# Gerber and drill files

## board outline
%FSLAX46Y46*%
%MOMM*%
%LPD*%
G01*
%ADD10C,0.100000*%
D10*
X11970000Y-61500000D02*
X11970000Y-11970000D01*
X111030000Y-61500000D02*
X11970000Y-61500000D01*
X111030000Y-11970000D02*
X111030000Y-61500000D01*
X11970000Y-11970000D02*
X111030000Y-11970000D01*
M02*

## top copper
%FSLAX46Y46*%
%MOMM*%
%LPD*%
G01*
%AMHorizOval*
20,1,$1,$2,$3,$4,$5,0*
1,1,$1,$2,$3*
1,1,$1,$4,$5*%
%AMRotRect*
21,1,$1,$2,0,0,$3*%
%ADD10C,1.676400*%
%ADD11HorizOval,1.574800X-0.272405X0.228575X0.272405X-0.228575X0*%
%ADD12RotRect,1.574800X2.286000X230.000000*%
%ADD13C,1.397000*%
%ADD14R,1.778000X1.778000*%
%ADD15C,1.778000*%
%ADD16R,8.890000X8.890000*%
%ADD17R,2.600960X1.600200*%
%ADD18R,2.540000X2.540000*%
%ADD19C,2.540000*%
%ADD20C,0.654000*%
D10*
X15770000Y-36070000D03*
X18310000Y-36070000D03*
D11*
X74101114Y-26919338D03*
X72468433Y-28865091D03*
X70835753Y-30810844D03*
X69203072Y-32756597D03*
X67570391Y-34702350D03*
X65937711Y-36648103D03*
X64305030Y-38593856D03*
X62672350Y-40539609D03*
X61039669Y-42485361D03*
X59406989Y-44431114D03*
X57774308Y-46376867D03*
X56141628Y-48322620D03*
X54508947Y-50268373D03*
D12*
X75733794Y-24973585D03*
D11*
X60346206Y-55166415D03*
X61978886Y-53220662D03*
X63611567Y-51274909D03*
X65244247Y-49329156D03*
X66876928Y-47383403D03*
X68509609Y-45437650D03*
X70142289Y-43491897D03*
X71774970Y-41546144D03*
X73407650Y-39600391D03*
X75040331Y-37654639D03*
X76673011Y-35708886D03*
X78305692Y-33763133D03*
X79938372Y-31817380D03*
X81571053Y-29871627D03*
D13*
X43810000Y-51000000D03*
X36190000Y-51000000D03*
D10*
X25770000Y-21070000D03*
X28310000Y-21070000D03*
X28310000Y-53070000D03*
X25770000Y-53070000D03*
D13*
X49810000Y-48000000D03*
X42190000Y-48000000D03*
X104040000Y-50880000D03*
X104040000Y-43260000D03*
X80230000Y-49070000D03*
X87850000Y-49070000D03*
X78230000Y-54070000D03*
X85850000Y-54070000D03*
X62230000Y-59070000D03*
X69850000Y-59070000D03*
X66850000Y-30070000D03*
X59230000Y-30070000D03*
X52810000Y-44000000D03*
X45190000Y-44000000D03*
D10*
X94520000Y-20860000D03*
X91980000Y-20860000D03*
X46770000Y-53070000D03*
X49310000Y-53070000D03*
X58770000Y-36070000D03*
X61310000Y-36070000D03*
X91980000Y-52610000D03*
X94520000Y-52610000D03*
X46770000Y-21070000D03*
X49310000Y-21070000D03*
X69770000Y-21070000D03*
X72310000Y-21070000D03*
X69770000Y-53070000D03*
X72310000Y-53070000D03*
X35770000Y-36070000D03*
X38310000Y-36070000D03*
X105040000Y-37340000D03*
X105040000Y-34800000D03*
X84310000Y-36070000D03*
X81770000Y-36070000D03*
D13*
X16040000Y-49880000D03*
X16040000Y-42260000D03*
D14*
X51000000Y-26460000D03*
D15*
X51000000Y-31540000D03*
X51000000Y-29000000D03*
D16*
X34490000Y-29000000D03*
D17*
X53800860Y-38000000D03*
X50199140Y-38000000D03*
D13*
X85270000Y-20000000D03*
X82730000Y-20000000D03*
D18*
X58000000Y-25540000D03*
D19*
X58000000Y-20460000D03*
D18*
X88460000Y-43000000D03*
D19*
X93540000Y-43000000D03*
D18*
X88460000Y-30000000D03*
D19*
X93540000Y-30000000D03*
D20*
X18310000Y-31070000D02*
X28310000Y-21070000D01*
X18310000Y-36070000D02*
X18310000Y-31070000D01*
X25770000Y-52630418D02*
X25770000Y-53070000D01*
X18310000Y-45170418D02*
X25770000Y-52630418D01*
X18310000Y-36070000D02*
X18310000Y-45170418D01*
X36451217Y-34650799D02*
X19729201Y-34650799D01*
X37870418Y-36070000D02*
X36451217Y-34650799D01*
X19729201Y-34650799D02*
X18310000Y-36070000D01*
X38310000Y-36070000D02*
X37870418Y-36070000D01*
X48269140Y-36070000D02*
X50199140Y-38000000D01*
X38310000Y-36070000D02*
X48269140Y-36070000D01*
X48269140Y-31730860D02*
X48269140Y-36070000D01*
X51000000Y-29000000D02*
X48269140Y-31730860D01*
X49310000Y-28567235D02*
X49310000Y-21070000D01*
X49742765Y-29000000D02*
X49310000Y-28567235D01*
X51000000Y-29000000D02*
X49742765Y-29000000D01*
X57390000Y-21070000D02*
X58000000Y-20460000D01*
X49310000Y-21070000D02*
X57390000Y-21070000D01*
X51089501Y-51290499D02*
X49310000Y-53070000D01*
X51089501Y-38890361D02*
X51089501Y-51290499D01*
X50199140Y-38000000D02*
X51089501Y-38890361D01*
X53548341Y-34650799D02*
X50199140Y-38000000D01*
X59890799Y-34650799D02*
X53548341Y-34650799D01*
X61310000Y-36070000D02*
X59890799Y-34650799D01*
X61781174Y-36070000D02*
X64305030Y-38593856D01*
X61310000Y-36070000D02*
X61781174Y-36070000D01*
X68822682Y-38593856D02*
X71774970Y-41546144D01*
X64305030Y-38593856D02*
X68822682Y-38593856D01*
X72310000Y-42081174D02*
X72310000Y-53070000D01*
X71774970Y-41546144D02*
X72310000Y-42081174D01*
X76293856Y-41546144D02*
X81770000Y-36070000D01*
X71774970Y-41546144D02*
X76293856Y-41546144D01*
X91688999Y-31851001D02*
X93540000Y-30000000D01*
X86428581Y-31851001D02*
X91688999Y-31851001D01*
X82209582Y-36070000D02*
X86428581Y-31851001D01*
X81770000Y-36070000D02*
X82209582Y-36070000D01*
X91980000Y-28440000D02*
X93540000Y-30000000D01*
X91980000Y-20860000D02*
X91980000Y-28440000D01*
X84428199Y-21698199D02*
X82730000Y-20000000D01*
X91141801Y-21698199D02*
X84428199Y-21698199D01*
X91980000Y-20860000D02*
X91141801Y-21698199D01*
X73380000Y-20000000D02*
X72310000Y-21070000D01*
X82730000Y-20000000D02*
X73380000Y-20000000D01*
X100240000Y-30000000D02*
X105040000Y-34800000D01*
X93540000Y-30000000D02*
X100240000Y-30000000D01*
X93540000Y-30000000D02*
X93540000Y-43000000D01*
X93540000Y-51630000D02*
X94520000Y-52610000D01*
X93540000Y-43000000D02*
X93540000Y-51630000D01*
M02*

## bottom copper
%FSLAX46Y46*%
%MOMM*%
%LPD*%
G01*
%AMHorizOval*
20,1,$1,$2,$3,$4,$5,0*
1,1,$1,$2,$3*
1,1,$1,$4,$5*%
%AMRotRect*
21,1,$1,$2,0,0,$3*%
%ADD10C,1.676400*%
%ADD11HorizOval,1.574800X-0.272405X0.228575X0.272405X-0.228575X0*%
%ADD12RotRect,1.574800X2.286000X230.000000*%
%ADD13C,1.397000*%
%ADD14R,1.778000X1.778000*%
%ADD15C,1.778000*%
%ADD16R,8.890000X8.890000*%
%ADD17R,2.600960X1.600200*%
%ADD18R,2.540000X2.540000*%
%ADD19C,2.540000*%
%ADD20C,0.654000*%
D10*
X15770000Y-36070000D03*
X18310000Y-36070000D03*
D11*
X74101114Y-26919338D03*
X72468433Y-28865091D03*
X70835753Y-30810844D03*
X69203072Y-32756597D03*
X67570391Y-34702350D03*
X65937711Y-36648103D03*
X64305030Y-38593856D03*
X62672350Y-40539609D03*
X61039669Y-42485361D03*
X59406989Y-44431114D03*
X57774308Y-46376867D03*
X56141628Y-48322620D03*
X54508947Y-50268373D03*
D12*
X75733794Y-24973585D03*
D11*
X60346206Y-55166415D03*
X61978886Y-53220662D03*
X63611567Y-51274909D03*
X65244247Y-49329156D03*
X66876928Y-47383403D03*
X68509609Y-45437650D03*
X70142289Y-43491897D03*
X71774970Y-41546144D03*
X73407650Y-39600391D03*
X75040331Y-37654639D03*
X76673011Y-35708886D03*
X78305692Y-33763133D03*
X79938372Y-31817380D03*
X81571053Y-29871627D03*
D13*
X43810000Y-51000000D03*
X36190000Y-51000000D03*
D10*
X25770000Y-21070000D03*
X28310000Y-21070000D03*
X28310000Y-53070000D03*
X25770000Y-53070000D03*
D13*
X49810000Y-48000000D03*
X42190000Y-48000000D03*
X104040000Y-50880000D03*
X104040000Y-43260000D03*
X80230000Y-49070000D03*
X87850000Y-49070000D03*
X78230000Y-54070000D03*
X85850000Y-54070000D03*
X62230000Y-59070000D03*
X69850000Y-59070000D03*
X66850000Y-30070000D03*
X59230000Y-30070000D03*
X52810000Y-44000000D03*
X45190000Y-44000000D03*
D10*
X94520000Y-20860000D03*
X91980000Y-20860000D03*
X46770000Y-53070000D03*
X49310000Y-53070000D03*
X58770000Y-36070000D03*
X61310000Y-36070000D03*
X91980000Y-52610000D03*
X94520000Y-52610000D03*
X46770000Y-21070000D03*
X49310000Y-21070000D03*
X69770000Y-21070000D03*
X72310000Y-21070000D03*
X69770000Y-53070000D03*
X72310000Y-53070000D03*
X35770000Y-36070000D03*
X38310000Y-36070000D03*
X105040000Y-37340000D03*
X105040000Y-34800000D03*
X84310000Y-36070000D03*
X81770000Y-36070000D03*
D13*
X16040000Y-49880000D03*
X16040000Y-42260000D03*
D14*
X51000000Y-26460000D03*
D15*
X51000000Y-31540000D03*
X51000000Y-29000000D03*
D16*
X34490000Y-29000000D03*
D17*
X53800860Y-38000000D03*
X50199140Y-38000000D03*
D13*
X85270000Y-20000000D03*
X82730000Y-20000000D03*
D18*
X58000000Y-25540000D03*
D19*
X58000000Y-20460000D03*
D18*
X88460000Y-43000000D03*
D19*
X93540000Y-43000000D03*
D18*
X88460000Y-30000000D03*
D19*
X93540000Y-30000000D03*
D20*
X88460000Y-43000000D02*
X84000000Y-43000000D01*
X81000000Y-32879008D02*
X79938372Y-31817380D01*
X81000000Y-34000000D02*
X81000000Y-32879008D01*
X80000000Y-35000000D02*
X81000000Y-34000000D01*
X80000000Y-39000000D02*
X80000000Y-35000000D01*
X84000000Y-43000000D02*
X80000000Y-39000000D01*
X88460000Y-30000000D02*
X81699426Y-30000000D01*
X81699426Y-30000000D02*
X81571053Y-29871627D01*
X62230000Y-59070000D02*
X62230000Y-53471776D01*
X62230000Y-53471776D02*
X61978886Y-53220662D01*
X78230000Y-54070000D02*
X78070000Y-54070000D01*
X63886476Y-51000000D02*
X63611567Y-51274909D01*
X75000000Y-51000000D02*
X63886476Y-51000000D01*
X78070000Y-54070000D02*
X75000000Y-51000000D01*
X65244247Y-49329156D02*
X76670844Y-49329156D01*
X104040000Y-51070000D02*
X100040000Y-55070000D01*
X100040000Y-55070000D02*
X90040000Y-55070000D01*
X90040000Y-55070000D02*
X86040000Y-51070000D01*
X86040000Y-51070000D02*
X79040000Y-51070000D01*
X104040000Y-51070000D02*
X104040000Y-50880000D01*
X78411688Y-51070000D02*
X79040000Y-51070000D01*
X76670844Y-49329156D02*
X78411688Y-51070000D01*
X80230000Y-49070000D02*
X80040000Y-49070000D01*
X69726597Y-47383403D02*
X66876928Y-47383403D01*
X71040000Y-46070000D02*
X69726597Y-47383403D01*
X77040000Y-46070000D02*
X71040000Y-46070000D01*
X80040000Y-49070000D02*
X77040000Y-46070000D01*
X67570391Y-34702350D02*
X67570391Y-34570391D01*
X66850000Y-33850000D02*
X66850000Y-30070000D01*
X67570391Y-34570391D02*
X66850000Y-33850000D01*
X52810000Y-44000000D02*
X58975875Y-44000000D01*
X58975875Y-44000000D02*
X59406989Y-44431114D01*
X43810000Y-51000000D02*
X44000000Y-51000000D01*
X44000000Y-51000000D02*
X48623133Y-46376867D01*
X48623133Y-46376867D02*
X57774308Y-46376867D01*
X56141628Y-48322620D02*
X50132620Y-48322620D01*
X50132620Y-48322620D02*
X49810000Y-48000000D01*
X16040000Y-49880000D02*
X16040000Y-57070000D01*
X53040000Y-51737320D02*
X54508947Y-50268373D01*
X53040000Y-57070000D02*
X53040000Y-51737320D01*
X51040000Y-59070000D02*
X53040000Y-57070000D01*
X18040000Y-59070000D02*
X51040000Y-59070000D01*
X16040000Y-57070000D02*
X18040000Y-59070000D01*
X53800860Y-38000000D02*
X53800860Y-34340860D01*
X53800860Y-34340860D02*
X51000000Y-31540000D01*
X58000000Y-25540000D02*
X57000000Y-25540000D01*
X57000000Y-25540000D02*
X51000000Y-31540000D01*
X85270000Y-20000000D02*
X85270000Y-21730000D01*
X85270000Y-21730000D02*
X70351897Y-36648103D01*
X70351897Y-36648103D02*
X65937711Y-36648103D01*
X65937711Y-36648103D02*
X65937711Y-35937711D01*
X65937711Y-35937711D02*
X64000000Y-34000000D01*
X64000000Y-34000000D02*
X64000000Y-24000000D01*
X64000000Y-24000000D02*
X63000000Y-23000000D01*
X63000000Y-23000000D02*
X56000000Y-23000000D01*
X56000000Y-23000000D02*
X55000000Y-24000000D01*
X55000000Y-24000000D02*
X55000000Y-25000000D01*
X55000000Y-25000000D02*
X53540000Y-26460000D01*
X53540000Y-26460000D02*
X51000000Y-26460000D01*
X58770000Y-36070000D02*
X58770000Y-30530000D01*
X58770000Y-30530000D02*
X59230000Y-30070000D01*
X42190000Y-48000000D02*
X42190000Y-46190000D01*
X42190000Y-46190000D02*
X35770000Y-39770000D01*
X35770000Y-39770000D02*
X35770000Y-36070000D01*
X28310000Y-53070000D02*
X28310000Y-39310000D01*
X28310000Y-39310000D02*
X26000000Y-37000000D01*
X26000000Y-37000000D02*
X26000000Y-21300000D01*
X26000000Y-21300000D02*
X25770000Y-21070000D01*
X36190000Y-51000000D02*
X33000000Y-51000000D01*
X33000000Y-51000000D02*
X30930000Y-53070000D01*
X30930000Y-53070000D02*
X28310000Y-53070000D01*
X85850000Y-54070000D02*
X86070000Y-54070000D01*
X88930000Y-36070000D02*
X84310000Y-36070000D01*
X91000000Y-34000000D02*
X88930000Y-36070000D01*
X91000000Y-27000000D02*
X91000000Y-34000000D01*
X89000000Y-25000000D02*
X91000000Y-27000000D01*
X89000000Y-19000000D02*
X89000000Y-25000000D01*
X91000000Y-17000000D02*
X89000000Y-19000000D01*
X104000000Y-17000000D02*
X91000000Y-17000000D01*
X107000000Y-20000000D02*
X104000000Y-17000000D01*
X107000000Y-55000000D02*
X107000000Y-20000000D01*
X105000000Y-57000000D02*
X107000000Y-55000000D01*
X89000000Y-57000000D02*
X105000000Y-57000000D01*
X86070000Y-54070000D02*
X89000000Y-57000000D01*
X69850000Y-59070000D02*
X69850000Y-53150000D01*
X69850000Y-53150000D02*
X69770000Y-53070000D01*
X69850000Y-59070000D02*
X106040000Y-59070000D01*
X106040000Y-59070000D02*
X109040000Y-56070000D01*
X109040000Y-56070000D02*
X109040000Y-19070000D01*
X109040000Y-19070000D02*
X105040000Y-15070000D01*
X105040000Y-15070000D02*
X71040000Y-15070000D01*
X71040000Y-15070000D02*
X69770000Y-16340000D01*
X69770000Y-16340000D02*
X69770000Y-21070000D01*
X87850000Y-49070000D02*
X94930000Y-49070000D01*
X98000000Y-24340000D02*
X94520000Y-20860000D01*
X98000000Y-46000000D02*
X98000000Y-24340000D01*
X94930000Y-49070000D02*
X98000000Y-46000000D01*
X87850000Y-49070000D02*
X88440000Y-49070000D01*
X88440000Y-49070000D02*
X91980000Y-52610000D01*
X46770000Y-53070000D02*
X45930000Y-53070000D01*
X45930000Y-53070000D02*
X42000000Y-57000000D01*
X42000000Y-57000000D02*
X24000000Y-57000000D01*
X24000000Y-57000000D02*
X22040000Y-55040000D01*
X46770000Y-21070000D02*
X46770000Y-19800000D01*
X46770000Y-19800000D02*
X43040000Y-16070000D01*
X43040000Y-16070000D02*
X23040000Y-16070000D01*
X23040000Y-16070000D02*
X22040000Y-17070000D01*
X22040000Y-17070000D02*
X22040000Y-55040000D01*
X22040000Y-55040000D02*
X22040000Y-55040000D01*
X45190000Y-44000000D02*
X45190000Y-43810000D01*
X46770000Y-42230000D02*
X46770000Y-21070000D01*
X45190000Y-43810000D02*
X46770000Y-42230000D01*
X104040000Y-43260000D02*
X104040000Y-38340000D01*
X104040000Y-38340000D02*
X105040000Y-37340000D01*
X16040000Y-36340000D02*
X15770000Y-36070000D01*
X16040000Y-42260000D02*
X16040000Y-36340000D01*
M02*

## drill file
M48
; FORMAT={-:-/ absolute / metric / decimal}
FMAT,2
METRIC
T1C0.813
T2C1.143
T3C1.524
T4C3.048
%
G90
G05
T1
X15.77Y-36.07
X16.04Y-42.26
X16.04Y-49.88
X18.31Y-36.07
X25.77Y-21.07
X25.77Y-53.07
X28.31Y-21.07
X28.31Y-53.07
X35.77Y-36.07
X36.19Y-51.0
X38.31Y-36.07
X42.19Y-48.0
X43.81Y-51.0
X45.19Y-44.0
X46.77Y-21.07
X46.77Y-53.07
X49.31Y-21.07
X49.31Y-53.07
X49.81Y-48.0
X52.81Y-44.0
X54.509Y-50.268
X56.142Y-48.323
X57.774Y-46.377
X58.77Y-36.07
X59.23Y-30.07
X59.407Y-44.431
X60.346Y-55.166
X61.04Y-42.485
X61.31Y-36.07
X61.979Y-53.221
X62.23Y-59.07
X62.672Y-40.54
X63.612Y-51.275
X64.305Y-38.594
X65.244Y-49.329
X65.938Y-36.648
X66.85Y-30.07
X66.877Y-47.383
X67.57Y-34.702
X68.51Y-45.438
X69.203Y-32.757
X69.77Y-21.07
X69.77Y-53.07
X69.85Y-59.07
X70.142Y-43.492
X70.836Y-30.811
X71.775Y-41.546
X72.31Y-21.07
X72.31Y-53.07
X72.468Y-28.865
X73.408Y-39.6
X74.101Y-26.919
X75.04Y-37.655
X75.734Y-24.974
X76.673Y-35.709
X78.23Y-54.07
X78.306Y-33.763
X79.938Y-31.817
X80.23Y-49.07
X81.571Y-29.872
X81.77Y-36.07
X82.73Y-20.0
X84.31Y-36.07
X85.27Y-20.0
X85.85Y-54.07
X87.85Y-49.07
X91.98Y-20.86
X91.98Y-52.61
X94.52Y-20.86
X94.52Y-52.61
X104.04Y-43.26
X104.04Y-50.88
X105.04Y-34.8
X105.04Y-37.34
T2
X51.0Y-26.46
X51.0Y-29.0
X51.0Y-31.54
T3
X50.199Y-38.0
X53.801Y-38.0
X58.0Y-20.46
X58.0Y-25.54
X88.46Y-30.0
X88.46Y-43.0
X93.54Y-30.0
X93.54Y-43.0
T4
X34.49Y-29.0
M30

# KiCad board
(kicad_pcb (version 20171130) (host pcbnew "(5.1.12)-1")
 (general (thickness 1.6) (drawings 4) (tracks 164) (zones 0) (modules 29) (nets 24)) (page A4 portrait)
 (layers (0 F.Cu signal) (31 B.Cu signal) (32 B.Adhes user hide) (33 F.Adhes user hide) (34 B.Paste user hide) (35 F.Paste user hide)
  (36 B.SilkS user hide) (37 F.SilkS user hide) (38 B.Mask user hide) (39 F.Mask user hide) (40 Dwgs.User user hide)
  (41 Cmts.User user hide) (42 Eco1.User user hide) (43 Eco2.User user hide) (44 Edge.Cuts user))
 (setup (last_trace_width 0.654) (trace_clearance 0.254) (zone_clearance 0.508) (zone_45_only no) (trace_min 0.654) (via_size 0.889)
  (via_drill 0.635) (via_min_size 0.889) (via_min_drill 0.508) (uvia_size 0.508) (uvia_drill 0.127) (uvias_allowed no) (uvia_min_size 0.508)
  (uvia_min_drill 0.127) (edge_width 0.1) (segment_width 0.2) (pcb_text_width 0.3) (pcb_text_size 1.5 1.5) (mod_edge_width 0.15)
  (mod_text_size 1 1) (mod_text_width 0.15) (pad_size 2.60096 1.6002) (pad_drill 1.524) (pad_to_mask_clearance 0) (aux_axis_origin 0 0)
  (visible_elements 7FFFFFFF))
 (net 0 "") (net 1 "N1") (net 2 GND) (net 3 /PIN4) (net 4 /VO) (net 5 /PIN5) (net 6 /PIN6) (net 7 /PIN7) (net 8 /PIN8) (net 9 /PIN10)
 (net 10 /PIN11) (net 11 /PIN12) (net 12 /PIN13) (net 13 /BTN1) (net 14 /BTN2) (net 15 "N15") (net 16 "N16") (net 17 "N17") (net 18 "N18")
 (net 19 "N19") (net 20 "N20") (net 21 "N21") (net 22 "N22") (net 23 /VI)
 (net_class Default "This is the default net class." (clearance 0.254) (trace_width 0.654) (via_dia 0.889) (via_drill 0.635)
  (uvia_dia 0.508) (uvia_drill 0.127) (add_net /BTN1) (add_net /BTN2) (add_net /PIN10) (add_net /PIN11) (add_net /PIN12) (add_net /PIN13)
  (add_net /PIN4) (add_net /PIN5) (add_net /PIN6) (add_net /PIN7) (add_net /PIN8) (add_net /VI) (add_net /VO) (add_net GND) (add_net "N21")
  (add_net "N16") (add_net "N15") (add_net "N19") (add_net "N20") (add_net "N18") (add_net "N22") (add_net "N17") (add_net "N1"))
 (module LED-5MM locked (layer B.Cu) (at 17.04 36.07)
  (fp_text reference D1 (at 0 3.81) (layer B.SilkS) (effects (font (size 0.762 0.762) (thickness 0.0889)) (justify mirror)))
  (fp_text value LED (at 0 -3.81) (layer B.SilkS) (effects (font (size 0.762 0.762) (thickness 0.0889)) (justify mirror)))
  (pad 1 thru_hole circle (at -1.27 0) (size 1.6764 1.6764) (drill 0.8128) (layers *.Cu *.Mask B.SilkS) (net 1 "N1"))
  (pad 2 thru_hole circle (at 1.27 0) (size 1.6764 1.6764) (drill 0.8128) (layers *.Cu *.Mask B.SilkS) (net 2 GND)))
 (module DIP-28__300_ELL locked (layer F.Cu) (at 68.04 40.07 230)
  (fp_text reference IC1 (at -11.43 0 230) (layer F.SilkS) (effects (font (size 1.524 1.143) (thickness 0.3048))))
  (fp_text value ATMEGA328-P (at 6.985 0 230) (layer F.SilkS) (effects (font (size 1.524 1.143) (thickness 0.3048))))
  (pad 2 thru_hole oval (at -13.97 3.81 230) (size 1.5748 2.286) (drill 0.8128) (layers *.Cu *.Mask F.SilkS))
  (pad 3 thru_hole oval (at -11.43 3.81 230) (size 1.5748 2.286) (drill 0.8128) (layers *.Cu *.Mask F.SilkS))
  (pad 4 thru_hole oval (at -8.89 3.81 230) (size 1.5748 2.286) (drill 0.8128) (layers *.Cu *.Mask F.SilkS))
  (pad 5 thru_hole oval (at -6.35 3.81 230) (size 1.5748 2.286) (drill 0.8128) (layers *.Cu *.Mask F.SilkS))
  (pad 6 thru_hole oval (at -3.81 3.81 230) (size 1.5748 2.286) (drill 0.8128) (layers *.Cu *.Mask F.SilkS) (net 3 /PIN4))
  (pad 7 thru_hole oval (at -1.27 3.81 230) (size 1.5748 2.286) (drill 0.8128) (layers *.Cu *.Mask F.SilkS) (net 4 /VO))
  (pad 8 thru_hole oval (at 1.27 3.81 230) (size 1.5748 2.286) (drill 0.8128) (layers *.Cu *.Mask F.SilkS) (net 2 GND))
  (pad 9 thru_hole oval (at 3.81 3.81 230) (size 1.5748 2.286) (drill 0.8128) (layers *.Cu *.Mask F.SilkS))
  (pad 10 thru_hole oval (at 6.35 3.81 230) (size 1.5748 2.286) (drill 0.8128) (layers *.Cu *.Mask F.SilkS))
  (pad 11 thru_hole oval (at 8.89 3.81 230) (size 1.5748 2.286) (drill 0.8128) (layers *.Cu *.Mask F.SilkS) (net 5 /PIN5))
  (pad 12 thru_hole oval (at 11.43 3.81 230) (size 1.5748 2.286) (drill 0.8128) (layers *.Cu *.Mask F.SilkS) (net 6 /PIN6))
  (pad 13 thru_hole oval (at 13.97 3.81 230) (size 1.5748 2.286) (drill 0.8128) (layers *.Cu *.Mask F.SilkS) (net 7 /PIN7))
  (pad 14 thru_hole oval (at 16.51 3.81 230) (size 1.5748 2.286) (drill 0.8128) (layers *.Cu *.Mask F.SilkS) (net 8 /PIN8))
  (pad 1 thru_hole rect (at -16.51 3.81 230) (size 1.5748 2.286) (drill 0.8128) (layers *.Cu *.Mask F.SilkS))
  (pad 15 thru_hole oval (at 16.51 -3.81 230) (size 1.5748 2.286) (drill 0.8128) (layers *.Cu *.Mask F.SilkS))
  (pad 16 thru_hole oval (at 13.97 -3.81 230) (size 1.5748 2.286) (drill 0.8128) (layers *.Cu *.Mask F.SilkS) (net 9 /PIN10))
  (pad 17 thru_hole oval (at 11.43 -3.81 230) (size 1.5748 2.286) (drill 0.8128) (layers *.Cu *.Mask F.SilkS) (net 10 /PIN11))
  (pad 18 thru_hole oval (at 8.89 -3.81 230) (size 1.5748 2.286) (drill 0.8128) (layers *.Cu *.Mask F.SilkS) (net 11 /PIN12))
  (pad 19 thru_hole oval (at 6.35 -3.81 230) (size 1.5748 2.286) (drill 0.8128) (layers *.Cu *.Mask F.SilkS) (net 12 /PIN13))
  (pad 20 thru_hole oval (at 3.81 -3.81 230) (size 1.5748 2.286) (drill 0.8128) (layers *.Cu *.Mask F.SilkS))
  (pad 21 thru_hole oval (at 1.27 -3.81 230) (size 1.5748 2.286) (drill 0.8128) (layers *.Cu *.Mask F.SilkS))
  (pad 22 thru_hole oval (at -1.27 -3.81 230) (size 1.5748 2.286) (drill 0.8128) (layers *.Cu *.Mask F.SilkS) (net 2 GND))
  (pad 23 thru_hole oval (at -3.81 -3.81 230) (size 1.5748 2.286) (drill 0.8128) (layers *.Cu *.Mask F.SilkS))
  (pad 24 thru_hole oval (at -6.35 -3.81 230) (size 1.5748 2.286) (drill 0.8128) (layers *.Cu *.Mask F.SilkS))
  (pad 25 thru_hole oval (at -8.89 -3.81 230) (size 1.5748 2.286) (drill 0.8128) (layers *.Cu *.Mask F.SilkS))
  (pad 26 thru_hole oval (at -11.43 -3.81 230) (size 1.5748 2.286) (drill 0.8128) (layers *.Cu *.Mask F.SilkS))
  (pad 27 thru_hole oval (at -13.97 -3.81 230) (size 1.5748 2.286) (drill 0.8128) (layers *.Cu *.Mask F.SilkS) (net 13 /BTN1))
  (pad 28 thru_hole oval (at -16.51 -3.81 230) (size 1.5748 2.286) (drill 0.8128) (layers *.Cu *.Mask F.SilkS) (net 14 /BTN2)))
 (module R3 (layer F.Cu) (at 40 51 180) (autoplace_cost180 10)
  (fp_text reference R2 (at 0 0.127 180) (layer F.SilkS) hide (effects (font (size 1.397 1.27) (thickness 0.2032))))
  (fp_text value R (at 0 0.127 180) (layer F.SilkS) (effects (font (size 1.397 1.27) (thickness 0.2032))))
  (pad 1 thru_hole circle (at -3.81 0 180) (size 1.397 1.397) (drill 0.8128) (layers *.Cu *.Mask F.SilkS) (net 6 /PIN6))
  (pad 2 thru_hole circle (at 3.81 0 180) (size 1.397 1.397) (drill 0.8128) (layers *.Cu *.Mask F.SilkS) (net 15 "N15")))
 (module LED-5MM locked (layer B.Cu) (at 27.04 21.07)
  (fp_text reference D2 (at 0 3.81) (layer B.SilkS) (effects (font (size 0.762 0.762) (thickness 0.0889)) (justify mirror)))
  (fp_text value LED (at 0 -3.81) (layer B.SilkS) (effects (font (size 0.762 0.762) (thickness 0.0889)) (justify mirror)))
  (pad 1 thru_hole circle (at -1.27 0) (size 1.6764 1.6764) (drill 0.8128) (layers *.Cu *.Mask B.SilkS) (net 15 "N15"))
  (pad 2 thru_hole circle (at 1.27 0) (size 1.6764 1.6764) (drill 0.8128) (layers *.Cu *.Mask B.SilkS) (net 2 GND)))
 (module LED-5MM (layer B.Cu) (at 27.04 53.07 180)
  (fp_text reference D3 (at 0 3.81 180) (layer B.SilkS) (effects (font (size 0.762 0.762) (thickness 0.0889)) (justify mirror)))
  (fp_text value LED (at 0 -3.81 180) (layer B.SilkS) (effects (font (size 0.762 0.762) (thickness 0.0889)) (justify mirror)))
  (pad 1 thru_hole circle (at -1.27 0 180) (size 1.6764 1.6764) (drill 0.8128) (layers *.Cu *.Mask B.SilkS) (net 15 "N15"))
  (pad 2 thru_hole circle (at 1.27 0 180) (size 1.6764 1.6764) (drill 0.8128) (layers *.Cu *.Mask B.SilkS) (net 2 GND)))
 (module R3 (layer F.Cu) (at 46 48 180) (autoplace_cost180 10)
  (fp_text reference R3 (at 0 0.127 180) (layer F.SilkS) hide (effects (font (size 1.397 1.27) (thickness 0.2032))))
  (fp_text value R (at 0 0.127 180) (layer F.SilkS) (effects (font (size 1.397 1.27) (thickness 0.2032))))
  (pad 1 thru_hole circle (at -3.81 0 180) (size 1.397 1.397) (drill 0.8128) (layers *.Cu *.Mask F.SilkS) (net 7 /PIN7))
  (pad 2 thru_hole circle (at 3.81 0 180) (size 1.397 1.397) (drill 0.8128) (layers *.Cu *.Mask F.SilkS) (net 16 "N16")))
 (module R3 (layer F.Cu) (at 104.04 47.07 90) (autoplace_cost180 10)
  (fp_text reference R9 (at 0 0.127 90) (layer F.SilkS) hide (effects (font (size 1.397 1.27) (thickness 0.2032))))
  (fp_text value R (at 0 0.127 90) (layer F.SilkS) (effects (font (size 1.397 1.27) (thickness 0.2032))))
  (pad 1 thru_hole circle (at -3.81 0 90) (size 1.397 1.397) (drill 0.8128) (layers *.Cu *.Mask F.SilkS) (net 11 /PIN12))
  (pad 2 thru_hole circle (at 3.81 0 90) (size 1.397 1.397) (drill 0.8128) (layers *.Cu *.Mask F.SilkS) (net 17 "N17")))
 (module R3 (layer F.Cu) (at 84.04 49.07) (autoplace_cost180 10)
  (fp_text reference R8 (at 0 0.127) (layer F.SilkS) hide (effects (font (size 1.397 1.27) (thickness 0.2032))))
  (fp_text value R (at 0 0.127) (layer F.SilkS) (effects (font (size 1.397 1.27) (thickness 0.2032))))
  (pad 1 thru_hole circle (at -3.81 0) (size 1.397 1.397) (drill 0.8128) (layers *.Cu *.Mask F.SilkS) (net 12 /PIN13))
  (pad 2 thru_hole circle (at 3.81 0) (size 1.397 1.397) (drill 0.8128) (layers *.Cu *.Mask F.SilkS) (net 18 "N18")))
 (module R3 (layer F.Cu) (at 82.04 54.07) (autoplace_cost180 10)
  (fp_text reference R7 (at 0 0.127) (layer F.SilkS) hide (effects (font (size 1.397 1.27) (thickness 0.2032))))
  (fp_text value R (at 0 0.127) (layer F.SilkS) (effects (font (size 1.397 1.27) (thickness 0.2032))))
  (pad 1 thru_hole circle (at -3.81 0) (size 1.397 1.397) (drill 0.8128) (layers *.Cu *.Mask F.SilkS) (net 10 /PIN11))
  (pad 2 thru_hole circle (at 3.81 0) (size 1.397 1.397) (drill 0.8128) (layers *.Cu *.Mask F.SilkS) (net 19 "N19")))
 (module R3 (layer F.Cu) (at 66.04 59.07) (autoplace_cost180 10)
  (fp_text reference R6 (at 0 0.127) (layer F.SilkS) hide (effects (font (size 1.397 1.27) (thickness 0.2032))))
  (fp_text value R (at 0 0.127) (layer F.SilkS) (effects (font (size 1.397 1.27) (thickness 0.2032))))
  (pad 1 thru_hole circle (at -3.81 0) (size 1.397 1.397) (drill 0.8128) (layers *.Cu *.Mask F.SilkS) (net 9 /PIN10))
  (pad 2 thru_hole circle (at 3.81 0) (size 1.397 1.397) (drill 0.8128) (layers *.Cu *.Mask F.SilkS) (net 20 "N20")))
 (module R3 (layer F.Cu) (at 63.04 30.07 180) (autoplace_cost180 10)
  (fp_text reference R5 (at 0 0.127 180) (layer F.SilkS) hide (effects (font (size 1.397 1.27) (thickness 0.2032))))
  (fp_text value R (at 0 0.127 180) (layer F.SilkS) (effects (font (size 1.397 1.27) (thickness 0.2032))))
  (pad 1 thru_hole circle (at -3.81 0 180) (size 1.397 1.397) (drill 0.8128) (layers *.Cu *.Mask F.SilkS) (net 3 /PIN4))
  (pad 2 thru_hole circle (at 3.81 0 180) (size 1.397 1.397) (drill 0.8128) (layers *.Cu *.Mask F.SilkS) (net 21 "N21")))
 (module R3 (layer F.Cu) (at 49 44 180) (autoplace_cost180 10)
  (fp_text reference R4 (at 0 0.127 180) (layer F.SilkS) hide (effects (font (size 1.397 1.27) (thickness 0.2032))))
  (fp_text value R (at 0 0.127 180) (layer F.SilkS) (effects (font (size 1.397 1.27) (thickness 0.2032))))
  (pad 1 thru_hole circle (at -3.81 0 180) (size 1.397 1.397) (drill 0.8128) (layers *.Cu *.Mask F.SilkS) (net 5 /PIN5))
  (pad 2 thru_hole circle (at 3.81 0 180) (size 1.397 1.397) (drill 0.8128) (layers *.Cu *.Mask F.SilkS) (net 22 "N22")))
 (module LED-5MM (layer B.Cu) (at 93.25 20.86 180)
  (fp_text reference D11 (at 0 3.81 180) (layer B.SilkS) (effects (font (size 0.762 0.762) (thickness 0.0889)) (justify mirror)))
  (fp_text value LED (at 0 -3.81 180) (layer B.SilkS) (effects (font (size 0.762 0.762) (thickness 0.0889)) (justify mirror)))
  (pad 1 thru_hole circle (at -1.27 0 180) (size 1.6764 1.6764) (drill 0.8128) (layers *.Cu *.Mask B.SilkS) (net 18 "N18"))
  (pad 2 thru_hole circle (at 1.27 0 180) (size 1.6764 1.6764) (drill 0.8128) (layers *.Cu *.Mask B.SilkS) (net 2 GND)))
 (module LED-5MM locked (layer B.Cu) (at 48.04 53.07)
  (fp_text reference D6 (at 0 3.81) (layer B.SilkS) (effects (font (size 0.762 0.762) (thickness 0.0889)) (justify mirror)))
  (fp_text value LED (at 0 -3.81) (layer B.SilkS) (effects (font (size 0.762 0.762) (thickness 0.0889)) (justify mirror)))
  (pad 1 thru_hole circle (at -1.27 0) (size 1.6764 1.6764) (drill 0.8128) (layers *.Cu *.Mask B.SilkS) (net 22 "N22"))
  (pad 2 thru_hole circle (at 1.27 0) (size 1.6764 1.6764) (drill 0.8128) (layers *.Cu *.Mask B.SilkS) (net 2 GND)))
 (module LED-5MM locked (layer B.Cu) (at 60.04 36.07)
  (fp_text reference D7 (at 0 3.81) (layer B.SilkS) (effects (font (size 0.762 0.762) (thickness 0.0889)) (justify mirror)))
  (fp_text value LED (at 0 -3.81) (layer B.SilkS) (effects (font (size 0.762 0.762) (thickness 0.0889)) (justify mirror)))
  (pad 1 thru_hole circle (at -1.27 0) (size 1.6764 1.6764) (drill 0.8128) (layers *.Cu *.Mask B.SilkS) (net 21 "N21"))
  (pad 2 thru_hole circle (at 1.27 0) (size 1.6764 1.6764) (drill 0.8128) (layers *.Cu *.Mask B.SilkS) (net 2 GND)))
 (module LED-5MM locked (layer B.Cu) (at 93.25 52.61)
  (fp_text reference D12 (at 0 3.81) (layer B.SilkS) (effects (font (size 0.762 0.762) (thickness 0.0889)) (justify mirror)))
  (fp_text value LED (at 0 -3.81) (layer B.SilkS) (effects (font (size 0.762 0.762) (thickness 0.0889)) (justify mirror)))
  (pad 1 thru_hole circle (at -1.27 0) (size 1.6764 1.6764) (drill 0.8128) (layers *.Cu *.Mask B.SilkS) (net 18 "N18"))
  (pad 2 thru_hole circle (at 1.27 0) (size 1.6764 1.6764) (drill 0.8128) (layers *.Cu *.Mask B.SilkS) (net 2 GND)))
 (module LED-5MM (layer B.Cu) (at 48.04 21.07)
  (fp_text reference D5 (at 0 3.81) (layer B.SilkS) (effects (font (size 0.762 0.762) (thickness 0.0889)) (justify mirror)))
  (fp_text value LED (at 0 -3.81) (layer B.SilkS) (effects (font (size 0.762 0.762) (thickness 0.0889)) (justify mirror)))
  (pad 1 thru_hole circle (at -1.27 0) (size 1.6764 1.6764) (drill 0.8128) (layers *.Cu *.Mask B.SilkS) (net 22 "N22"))
  (pad 2 thru_hole circle (at 1.27 0) (size 1.6764 1.6764) (drill 0.8128) (layers *.Cu *.Mask B.SilkS) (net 2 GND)))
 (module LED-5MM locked (layer B.Cu) (at 71.04 21.07)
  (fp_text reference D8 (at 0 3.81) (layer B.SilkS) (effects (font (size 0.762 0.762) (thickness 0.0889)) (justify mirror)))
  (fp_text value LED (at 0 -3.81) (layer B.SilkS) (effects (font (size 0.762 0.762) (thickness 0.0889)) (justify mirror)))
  (pad 1 thru_hole circle (at -1.27 0) (size 1.6764 1.6764) (drill 0.8128) (layers *.Cu *.Mask B.SilkS) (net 20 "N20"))
  (pad 2 thru_hole circle (at 1.27 0) (size 1.6764 1.6764) (drill 0.8128) (layers *.Cu *.Mask B.SilkS) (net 2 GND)))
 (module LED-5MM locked (layer B.Cu) (at 71.04 53.07)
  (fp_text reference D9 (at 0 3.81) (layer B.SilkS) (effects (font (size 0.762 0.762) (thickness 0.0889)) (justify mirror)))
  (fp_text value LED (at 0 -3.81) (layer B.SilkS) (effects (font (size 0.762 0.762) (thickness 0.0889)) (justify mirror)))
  (pad 1 thru_hole circle (at -1.27 0) (size 1.6764 1.6764) (drill 0.8128) (layers *.Cu *.Mask B.SilkS) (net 20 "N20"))
  (pad 2 thru_hole circle (at 1.27 0) (size 1.6764 1.6764) (drill 0.8128) (layers *.Cu *.Mask B.SilkS) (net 2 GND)))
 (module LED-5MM (layer B.Cu) (at 37.04 36.07)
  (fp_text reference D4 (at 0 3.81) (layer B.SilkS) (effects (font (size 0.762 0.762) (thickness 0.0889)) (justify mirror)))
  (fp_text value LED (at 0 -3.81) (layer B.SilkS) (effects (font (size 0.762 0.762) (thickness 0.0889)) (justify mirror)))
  (pad 1 thru_hole circle (at -1.27 0) (size 1.6764 1.6764) (drill 0.8128) (layers *.Cu *.Mask B.SilkS) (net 16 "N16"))
  (pad 2 thru_hole circle (at 1.27 0) (size 1.6764 1.6764) (drill 0.8128) (layers *.Cu *.Mask B.SilkS) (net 2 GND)))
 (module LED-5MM (layer B.Cu) (at 105.04 36.07 90)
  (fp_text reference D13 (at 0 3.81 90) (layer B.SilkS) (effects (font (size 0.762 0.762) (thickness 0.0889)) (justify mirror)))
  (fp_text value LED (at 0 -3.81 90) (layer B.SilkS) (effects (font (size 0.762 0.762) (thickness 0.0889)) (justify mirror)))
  (pad 1 thru_hole circle (at -1.27 0 90) (size 1.6764 1.6764) (drill 0.8128) (layers *.Cu *.Mask B.SilkS) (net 17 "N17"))
  (pad 2 thru_hole circle (at 1.27 0 90) (size 1.6764 1.6764) (drill 0.8128) (layers *.Cu *.Mask B.SilkS) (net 2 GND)))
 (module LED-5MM (layer B.Cu) (at 83.04 36.07 180)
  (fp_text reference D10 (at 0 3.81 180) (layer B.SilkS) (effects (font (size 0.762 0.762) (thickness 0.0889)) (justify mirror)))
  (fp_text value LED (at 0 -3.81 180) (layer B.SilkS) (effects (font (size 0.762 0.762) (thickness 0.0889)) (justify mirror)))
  (pad 1 thru_hole circle (at -1.27 0 180) (size 1.6764 1.6764) (drill 0.8128) (layers *.Cu *.Mask B.SilkS) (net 19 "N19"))
  (pad 2 thru_hole circle (at 1.27 0 180) (size 1.6764 1.6764) (drill 0.8128) (layers *.Cu *.Mask B.SilkS) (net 2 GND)))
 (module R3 (layer F.Cu) (at 16.04 46.07 90) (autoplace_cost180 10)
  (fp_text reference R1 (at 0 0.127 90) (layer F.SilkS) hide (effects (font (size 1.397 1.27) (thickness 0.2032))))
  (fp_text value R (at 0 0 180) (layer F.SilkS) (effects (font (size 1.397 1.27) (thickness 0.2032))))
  (pad 1 thru_hole circle (at -3.81 0 90) (size 1.397 1.397) (drill 0.8128) (layers *.Cu *.Mask F.SilkS) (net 8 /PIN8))
  (pad 2 thru_hole circle (at 3.81 0 90) (size 1.397 1.397) (drill 0.8128) (layers *.Cu *.Mask F.SilkS) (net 1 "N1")))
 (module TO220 (layer F.Cu) (at 51 29 180)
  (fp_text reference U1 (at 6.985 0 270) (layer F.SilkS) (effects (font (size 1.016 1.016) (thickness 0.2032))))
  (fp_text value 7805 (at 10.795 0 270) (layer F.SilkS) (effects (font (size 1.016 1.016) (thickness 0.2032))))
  (pad 1 thru_hole rect (at 0 2.54 180) (size 1.778 1.778) (drill 1.143) (layers *.Cu *.Mask F.SilkS) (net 4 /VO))
  (pad 2 thru_hole circle (at 0 -2.54 180) (size 1.778 1.778) (drill 1.143) (layers *.Cu *.Mask F.SilkS) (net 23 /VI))
  (pad 3 thru_hole circle (at 0 0 180) (size 1.778 1.778) (drill 1.143) (layers *.Cu *.Mask F.SilkS) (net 2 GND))
  (pad 4 thru_hole rect (at 16.51 0 180) (size 8.89 8.89) (drill 3.048) (layers *.Cu *.SilkS *.Mask)))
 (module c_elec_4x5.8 (layer F.Cu) (at 52 38)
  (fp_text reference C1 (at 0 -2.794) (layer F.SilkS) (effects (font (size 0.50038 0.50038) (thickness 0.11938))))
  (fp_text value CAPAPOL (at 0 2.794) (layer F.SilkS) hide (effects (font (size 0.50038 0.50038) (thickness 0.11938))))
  (pad 1 thru_hole rect (at 1.80086 0) (size 2.60096 1.6002) (drill 1.524) (layers *.Cu *.Mask F.SilkS) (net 23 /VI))
  (pad 2 thru_hole rect (at -1.80086 0) (size 2.60096 1.6002) (drill 1.524) (layers *.Cu *.Mask F.SilkS) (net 2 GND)))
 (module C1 (layer F.Cu) (at 84 20 180)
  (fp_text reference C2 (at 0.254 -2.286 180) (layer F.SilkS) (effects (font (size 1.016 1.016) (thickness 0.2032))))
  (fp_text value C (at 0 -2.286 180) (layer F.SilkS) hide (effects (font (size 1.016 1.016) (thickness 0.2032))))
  (pad 1 thru_hole circle (at -1.27 0 180) (size 1.397 1.397) (drill 0.8128) (layers *.Cu *.Mask F.SilkS) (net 4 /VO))
  (pad 2 thru_hole circle (at 1.27 0 180) (size 1.397 1.397) (drill 0.8128) (layers *.Cu *.Mask F.SilkS) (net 2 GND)))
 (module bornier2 (layer F.Cu) (at 58 23 90)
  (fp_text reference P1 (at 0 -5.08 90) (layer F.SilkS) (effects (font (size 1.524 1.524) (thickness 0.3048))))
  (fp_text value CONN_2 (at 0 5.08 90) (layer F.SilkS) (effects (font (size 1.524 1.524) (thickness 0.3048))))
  (pad 1 thru_hole rect (at -2.54 0 90) (size 2.54 2.54) (drill 1.524) (layers *.Cu *.Mask F.SilkS) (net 23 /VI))
  (pad 2 thru_hole circle (at 2.54 0 90) (size 2.54 2.54) (drill 1.524) (layers *.Cu *.Mask F.SilkS) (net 2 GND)))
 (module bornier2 (layer F.Cu) (at 91 43)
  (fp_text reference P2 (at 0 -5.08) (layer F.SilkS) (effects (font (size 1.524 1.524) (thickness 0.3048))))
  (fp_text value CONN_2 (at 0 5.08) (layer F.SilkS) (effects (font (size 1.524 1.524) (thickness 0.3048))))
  (pad 1 thru_hole rect (at -2.54 0) (size 2.54 2.54) (drill 1.524) (layers *.Cu *.Mask F.SilkS) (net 13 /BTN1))
  (pad 2 thru_hole circle (at 2.54 0) (size 2.54 2.54) (drill 1.524) (layers *.Cu *.Mask F.SilkS) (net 2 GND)))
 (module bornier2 (layer F.Cu) (at 91 30)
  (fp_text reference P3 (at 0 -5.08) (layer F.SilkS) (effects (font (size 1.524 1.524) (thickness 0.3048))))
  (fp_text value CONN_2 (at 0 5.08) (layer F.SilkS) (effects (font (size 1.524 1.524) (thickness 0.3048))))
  (pad 1 thru_hole rect (at -2.54 0) (size 2.54 2.54) (drill 1.524) (layers *.Cu *.Mask F.SilkS) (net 14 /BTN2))
  (pad 2 thru_hole circle (at 2.54 0) (size 2.54 2.54) (drill 1.524) (layers *.Cu *.Mask F.SilkS) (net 2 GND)))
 (gr_line (start 11.97 61.5) (end 11.97 11.97) (angle 90) (layer Edge.Cuts) (width 0.1))
 (gr_line (start 111.03 61.5) (end 11.97 61.5) (angle 90) (layer Edge.Cuts) (width 0.1))
 (gr_line (start 111.03 11.97) (end 111.03 61.5) (angle 90) (layer Edge.Cuts) (width 0.1))
 (gr_line (start 11.97 11.97) (end 111.03 11.97) (angle 90) (layer Edge.Cuts) (width 0.1))
 (segment (start 88.46 43) (end 84 43) (width 0.654) (layer B.Cu) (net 13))
 (segment (start 81 32.879008) (end 79.938372 31.81738) (width 0.654) (layer B.Cu) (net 13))
 (segment (start 81 34) (end 81 32.879008) (width 0.654) (layer B.Cu) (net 13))
 (segment (start 80 35) (end 81 34) (width 0.654) (layer B.Cu) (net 13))
 (segment (start 80 39) (end 80 35) (width 0.654) (layer B.Cu) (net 13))
 (segment (start 84 43) (end 80 39) (width 0.654) (layer B.Cu) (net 13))
 (segment (start 88.46 30) (end 81.699426 30) (width 0.654) (layer B.Cu) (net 14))
 (segment (start 81.699426 30) (end 81.571053 29.871627) (width 0.654) (layer B.Cu) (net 14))
 (segment (start 62.23 59.07) (end 62.23 53.471776) (width 0.654) (layer B.Cu) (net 9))
 (segment (start 62.23 53.471776) (end 61.978886 53.220662) (width 0.654) (layer B.Cu) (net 9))
 (segment (start 78.23 54.07) (end 78.07 54.07) (width 0.654) (layer B.Cu) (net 10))
 (segment (start 63.886476 51) (end 63.611567 51.274909) (width 0.654) (layer B.Cu) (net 10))
 (segment (start 75 51) (end 63.886476 51) (width 0.654) (layer B.Cu) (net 10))
 (segment (start 78.07 54.07) (end 75 51) (width 0.654) (layer B.Cu) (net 10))
 (segment (start 65.244247 49.329156) (end 76.670844 49.329156) (width 0.654) (layer B.Cu) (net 11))
 (segment (start 104.04 51.07) (end 100.04 55.07) (width 0.654) (layer B.Cu) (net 11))
 (segment (start 100.04 55.07) (end 90.04 55.07) (width 0.654) (layer B.Cu) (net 11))
 (segment (start 90.04 55.07) (end 86.04 51.07) (width 0.654) (layer B.Cu) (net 11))
 (segment (start 86.04 51.07) (end 79.04 51.07) (width 0.654) (layer B.Cu) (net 11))
 (segment (start 104.04 51.07) (end 104.04 50.88) (width 0.654) (layer B.Cu) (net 11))
 (segment (start 78.411688 51.07) (end 79.04 51.07) (width 0.654) (layer B.Cu) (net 11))
 (segment (start 76.670844 49.329156) (end 78.411688 51.07) (width 0.654) (layer B.Cu) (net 11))
 (segment (start 80.23 49.07) (end 80.04 49.07) (width 0.654) (layer B.Cu) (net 12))
 (segment (start 69.726597 47.383403) (end 66.876928 47.383403) (width 0.654) (layer B.Cu) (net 12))
 (segment (start 71.04 46.07) (end 69.726597 47.383403) (width 0.654) (layer B.Cu) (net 12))
 (segment (start 77.04 46.07) (end 71.04 46.07) (width 0.654) (layer B.Cu) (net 12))
 (segment (start 80.04 49.07) (end 77.04 46.07) (width 0.654) (layer B.Cu) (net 12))
 (segment (start 67.570391 34.70235) (end 67.570391 34.570391) (width 0.654) (layer B.Cu) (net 3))
 (segment (start 66.85 33.85) (end 66.85 30.07) (width 0.654) (layer B.Cu) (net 3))
 (segment (start 67.570391 34.570391) (end 66.85 33.85) (width 0.654) (layer B.Cu) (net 3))
 (segment (start 52.81 44) (end 58.975875 44) (width 0.654) (layer B.Cu) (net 5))
 (segment (start 58.975875 44) (end 59.406989 44.431114) (width 0.654) (layer B.Cu) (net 5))
 (segment (start 43.81 51) (end 44 51) (width 0.654) (layer B.Cu) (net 6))
 (segment (start 44 51) (end 48.623133 46.376867) (width 0.654) (layer B.Cu) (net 6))
 (segment (start 48.623133 46.376867) (end 57.774308 46.376867) (width 0.654) (layer B.Cu) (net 6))
 (segment (start 56.141628 48.32262) (end 50.13262 48.32262) (width 0.654) (layer B.Cu) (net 7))
 (segment (start 50.13262 48.32262) (end 49.81 48) (width 0.654) (layer B.Cu) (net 7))
 (segment (start 16.04 49.88) (end 16.04 57.07) (width 0.654) (layer B.Cu) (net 8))
 (segment (start 53.04 51.73732) (end 54.508947 50.268373) (width 0.654) (layer B.Cu) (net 8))
 (segment (start 53.04 57.07) (end 53.04 51.73732) (width 0.654) (layer B.Cu) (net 8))
 (segment (start 51.04 59.07) (end 53.04 57.07) (width 0.654) (layer B.Cu) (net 8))
 (segment (start 18.04 59.07) (end 51.04 59.07) (width 0.654) (layer B.Cu) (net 8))
 (segment (start 16.04 57.07) (end 18.04 59.07) (width 0.654) (layer B.Cu) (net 8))
 (segment (start 53.80086 38) (end 53.80086 34.34086) (width 0.654) (layer B.Cu) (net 23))
 (segment (start 53.80086 34.34086) (end 51 31.54) (width 0.654) (layer B.Cu) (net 23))
 (segment (start 58 25.54) (end 57 25.54) (width 0.654) (layer B.Cu) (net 23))
 (segment (start 57 25.54) (end 51 31.54) (width 0.654) (layer B.Cu) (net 23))
 (segment (start 85.27 20) (end 85.27 21.73) (width 0.654) (layer B.Cu) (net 4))
 (segment (start 85.27 21.73) (end 70.351897 36.648103) (width 0.654) (layer B.Cu) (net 4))
 (segment (start 70.351897 36.648103) (end 65.937711 36.648103) (width 0.654) (layer B.Cu) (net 4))
 (segment (start 65.937711 36.648103) (end 65.937711 35.937711) (width 0.654) (layer B.Cu) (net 4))
 (segment (start 65.937711 35.937711) (end 64 34) (width 0.654) (layer B.Cu) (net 4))
 (segment (start 64 34) (end 64 24) (width 0.654) (layer B.Cu) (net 4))
 (segment (start 64 24) (end 63 23) (width 0.654) (layer B.Cu) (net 4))
 (segment (start 63 23) (end 56 23) (width 0.654) (layer B.Cu) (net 4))
 (segment (start 56 23) (end 55 24) (width 0.654) (layer B.Cu) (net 4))
 (segment (start 55 24) (end 55 25) (width 0.654) (layer B.Cu) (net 4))
 (segment (start 55 25) (end 53.54 26.46) (width 0.654) (layer B.Cu) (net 4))
 (segment (start 53.54 26.46) (end 51 26.46) (width 0.654) (layer B.Cu) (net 4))
 (segment (start 18.31 31.07) (end 28.31 21.07) (width 0.654) (layer F.Cu) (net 2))
 (segment (start 18.31 36.07) (end 18.31 31.07) (width 0.654) (layer F.Cu) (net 2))
 (segment (start 25.77 52.630418) (end 25.77 53.07) (width 0.654) (layer F.Cu) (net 2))
 (segment (start 18.31 45.170418) (end 25.77 52.630418) (width 0.654) (layer F.Cu) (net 2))
 (segment (start 18.31 36.07) (end 18.31 45.170418) (width 0.654) (layer F.Cu) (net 2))
 (segment (start 36.451217 34.650799) (end 19.729201 34.650799) (width 0.654) (layer F.Cu) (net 2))
 (segment (start 37.870418 36.07) (end 36.451217 34.650799) (width 0.654) (layer F.Cu) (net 2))
 (segment (start 19.729201 34.650799) (end 18.31 36.07) (width 0.654) (layer F.Cu) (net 2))
 (segment (start 38.31 36.07) (end 37.870418 36.07) (width 0.654) (layer F.Cu) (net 2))
 (segment (start 48.26914 36.07) (end 50.19914 38) (width 0.654) (layer F.Cu) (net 2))
 (segment (start 38.31 36.07) (end 48.26914 36.07) (width 0.654) (layer F.Cu) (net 2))
 (segment (start 48.26914 31.73086) (end 48.26914 36.07) (width 0.654) (layer F.Cu) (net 2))
 (segment (start 51 29) (end 48.26914 31.73086) (width 0.654) (layer F.Cu) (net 2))
 (segment (start 49.31 28.567235) (end 49.31 21.07) (width 0.654) (layer F.Cu) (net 2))
 (segment (start 49.742765 29) (end 49.31 28.567235) (width 0.654) (layer F.Cu) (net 2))
 (segment (start 51 29) (end 49.742765 29) (width 0.654) (layer F.Cu) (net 2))
 (segment (start 57.39 21.07) (end 58 20.46) (width 0.654) (layer F.Cu) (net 2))
 (segment (start 49.31 21.07) (end 57.39 21.07) (width 0.654) (layer F.Cu) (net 2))
 (segment (start 51.089501 51.290499) (end 49.31 53.07) (width 0.654) (layer F.Cu) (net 2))
 (segment (start 51.089501 38.890361) (end 51.089501 51.290499) (width 0.654) (layer F.Cu) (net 2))
 (segment (start 50.19914 38) (end 51.089501 38.890361) (width 0.654) (layer F.Cu) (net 2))
 (segment (start 53.548341 34.650799) (end 50.19914 38) (width 0.654) (layer F.Cu) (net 2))
 (segment (start 59.890799 34.650799) (end 53.548341 34.650799) (width 0.654) (layer F.Cu) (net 2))
 (segment (start 61.31 36.07) (end 59.890799 34.650799) (width 0.654) (layer F.Cu) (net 2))
 (segment (start 61.781174 36.07) (end 64.30503 38.593856) (width 0.654) (layer F.Cu) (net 2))
 (segment (start 61.31 36.07) (end 61.781174 36.07) (width 0.654) (layer F.Cu) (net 2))
 (segment (start 68.822682 38.593856) (end 71.77497 41.546144) (width 0.654) (layer F.Cu) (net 2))
 (segment (start 64.30503 38.593856) (end 68.822682 38.593856) (width 0.654) (layer F.Cu) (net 2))
 (segment (start 72.31 42.081174) (end 72.31 53.07) (width 0.654) (layer F.Cu) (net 2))
 (segment (start 71.77497 41.546144) (end 72.31 42.081174) (width 0.654) (layer F.Cu) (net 2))
 (segment (start 76.293856 41.546144) (end 81.77 36.07) (width 0.654) (layer F.Cu) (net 2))
 (segment (start 71.77497 41.546144) (end 76.293856 41.546144) (width 0.654) (layer F.Cu) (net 2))
 (segment (start 91.688999 31.851001) (end 93.54 30) (width 0.654) (layer F.Cu) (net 2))
 (segment (start 86.428581 31.851001) (end 91.688999 31.851001) (width 0.654) (layer F.Cu) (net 2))
 (segment (start 82.209582 36.07) (end 86.428581 31.851001) (width 0.654) (layer F.Cu) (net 2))
 (segment (start 81.77 36.07) (end 82.209582 36.07) (width 0.654) (layer F.Cu) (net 2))
 (segment (start 91.98 28.44) (end 93.54 30) (width 0.654) (layer F.Cu) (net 2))
 (segment (start 91.98 20.86) (end 91.98 28.44) (width 0.654) (layer F.Cu) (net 2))
 (segment (start 84.428199 21.698199) (end 82.73 20) (width 0.654) (layer F.Cu) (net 2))
 (segment (start 91.141801 21.698199) (end 84.428199 21.698199) (width 0.654) (layer F.Cu) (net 2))
 (segment (start 91.98 20.86) (end 91.141801 21.698199) (width 0.654) (layer F.Cu) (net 2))
 (segment (start 73.38 20) (end 72.31 21.07) (width 0.654) (layer F.Cu) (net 2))
 (segment (start 82.73 20) (end 73.38 20) (width 0.654) (layer F.Cu) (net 2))
 (segment (start 100.24 30) (end 105.04 34.8) (width 0.654) (layer F.Cu) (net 2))
 (segment (start 93.54 30) (end 100.24 30) (width 0.654) (layer F.Cu) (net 2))
 (segment (start 93.54 30) (end 93.54 43) (width 0.654) (layer F.Cu) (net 2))
 (segment (start 93.54 51.63) (end 94.52 52.61) (width 0.654) (layer F.Cu) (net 2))
 (segment (start 93.54 43) (end 93.54 51.63) (width 0.654) (layer F.Cu) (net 2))
 (segment (start 58.77 36.07) (end 58.77 30.53) (width 0.654) (layer B.Cu) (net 21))
 (segment (start 58.77 30.53) (end 59.23 30.07) (width 0.654) (layer B.Cu) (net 21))
 (segment (start 42.19 48) (end 42.19 46.19) (width 0.654) (layer B.Cu) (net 16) (status 10))
 (segment (start 42.19 46.19) (end 35.77 39.77) (width 0.654) (layer B.Cu) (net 16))
 (segment (start 35.77 39.77) (end 35.77 36.07) (width 0.654) (layer B.Cu) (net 16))
 (segment (start 28.31 53.07) (end 28.31 39.31) (width 0.654) (layer B.Cu) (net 15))
 (segment (start 28.31 39.31) (end 26 37) (width 0.654) (layer B.Cu) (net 15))
 (segment (start 26 37) (end 26 21.3) (width 0.654) (layer B.Cu) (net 15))
 (segment (start 26 21.3) (end 25.77 21.07) (width 0.654) (layer B.Cu) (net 15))
 (segment (start 36.19 51) (end 33 51) (width 0.654) (layer B.Cu) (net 15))
 (segment (start 33 51) (end 30.93 53.07) (width 0.654) (layer B.Cu) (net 15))
 (segment (start 30.93 53.07) (end 28.31 53.07) (width 0.654) (layer B.Cu) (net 15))
 (segment (start 85.85 54.07) (end 86.07 54.07) (width 0.654) (layer B.Cu) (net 19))
 (segment (start 88.93 36.07) (end 84.31 36.07) (width 0.654) (layer B.Cu) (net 19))
 (segment (start 91 34) (end 88.93 36.07) (width 0.654) (layer B.Cu) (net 19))
 (segment (start 91 27) (end 91 34) (width 0.654) (layer B.Cu) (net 19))
 (segment (start 89 25) (end 91 27) (width 0.654) (layer B.Cu) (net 19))
 (segment (start 89 19) (end 89 25) (width 0.654) (layer B.Cu) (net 19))
 (segment (start 91 17) (end 89 19) (width 0.654) (layer B.Cu) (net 19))
 (segment (start 104 17) (end 91 17) (width 0.654) (layer B.Cu) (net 19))
 (segment (start 107 20) (end 104 17) (width 0.654) (layer B.Cu) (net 19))
 (segment (start 107 55) (end 107 20) (width 0.654) (layer B.Cu) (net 19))
 (segment (start 105 57) (end 107 55) (width 0.654) (layer B.Cu) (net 19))
 (segment (start 89 57) (end 105 57) (width 0.654) (layer B.Cu) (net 19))
 (segment (start 86.07 54.07) (end 89 57) (width 0.654) (layer B.Cu) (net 19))
 (segment (start 69.85 59.07) (end 69.85 53.15) (width 0.654) (layer B.Cu) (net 20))
 (segment (start 69.85 53.15) (end 69.77 53.07) (width 0.654) (layer B.Cu) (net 20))
 (segment (start 69.85 59.07) (end 106.04 59.07) (width 0.654) (layer B.Cu) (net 20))
 (segment (start 106.04 59.07) (end 109.04 56.07) (width 0.654) (layer B.Cu) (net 20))
 (segment (start 109.04 56.07) (end 109.04 19.07) (width 0.654) (layer B.Cu) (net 20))
 (segment (start 109.04 19.07) (end 105.04 15.07) (width 0.654) (layer B.Cu) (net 20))
 (segment (start 105.04 15.07) (end 71.04 15.07) (width 0.654) (layer B.Cu) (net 20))
 (segment (start 71.04 15.07) (end 69.77 16.34) (width 0.654) (layer B.Cu) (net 20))
 (segment (start 69.77 16.34) (end 69.77 21.07) (width 0.654) (layer B.Cu) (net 20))
 (segment (start 87.85 49.07) (end 94.93 49.07) (width 0.654) (layer B.Cu) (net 18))
 (segment (start 98 24.34) (end 94.52 20.86) (width 0.654) (layer B.Cu) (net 18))
 (segment (start 98 46) (end 98 24.34) (width 0.654) (layer B.Cu) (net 18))
 (segment (start 94.93 49.07) (end 98 46) (width 0.654) (layer B.Cu) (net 18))
 (segment (start 87.85 49.07) (end 88.44 49.07) (width 0.654) (layer B.Cu) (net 18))
 (segment (start 88.44 49.07) (end 91.98 52.61) (width 0.654) (layer B.Cu) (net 18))
 (segment (start 46.77 53.07) (end 45.93 53.07) (width 0.654) (layer B.Cu) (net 22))
 (segment (start 45.93 53.07) (end 42 57) (width 0.654) (layer B.Cu) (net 22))
 (segment (start 42 57) (end 24 57) (width 0.654) (layer B.Cu) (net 22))
 (segment (start 24 57) (end 22.04 55.04) (width 0.654) (layer B.Cu) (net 22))
 (segment (start 46.77 21.07) (end 46.77 19.8) (width 0.654) (layer B.Cu) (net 22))
 (segment (start 46.77 19.8) (end 43.04 16.07) (width 0.654) (layer B.Cu) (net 22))
 (segment (start 43.04 16.07) (end 23.04 16.07) (width 0.654) (layer B.Cu) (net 22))
 (segment (start 23.04 16.07) (end 22.04 17.07) (width 0.654) (layer B.Cu) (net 22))
 (segment (start 22.04 17.07) (end 22.04 55.04) (width 0.654) (layer B.Cu) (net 22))
 (segment (start 22.04 55.04) (end 22.04 55.04) (width 0.654) (layer B.Cu) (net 22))
 (segment (start 45.19 44) (end 45.19 43.81) (width 0.654) (layer B.Cu) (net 22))
 (segment (start 46.77 42.23) (end 46.77 21.07) (width 0.654) (layer B.Cu) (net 22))
 (segment (start 45.19 43.81) (end 46.77 42.23) (width 0.654) (layer B.Cu) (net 22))
 (segment (start 104.04 43.26) (end 104.04 38.34) (width 0.654) (layer B.Cu) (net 17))
 (segment (start 104.04 38.34) (end 105.04 37.34) (width 0.654) (layer B.Cu) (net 17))
 (segment (start 16.04 36.34) (end 15.77 36.07) (width 0.654) (layer B.Cu) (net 1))
 (segment (start 16.04 42.26) (end 16.04 36.34) (width 0.654) (layer B.Cu) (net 1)))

